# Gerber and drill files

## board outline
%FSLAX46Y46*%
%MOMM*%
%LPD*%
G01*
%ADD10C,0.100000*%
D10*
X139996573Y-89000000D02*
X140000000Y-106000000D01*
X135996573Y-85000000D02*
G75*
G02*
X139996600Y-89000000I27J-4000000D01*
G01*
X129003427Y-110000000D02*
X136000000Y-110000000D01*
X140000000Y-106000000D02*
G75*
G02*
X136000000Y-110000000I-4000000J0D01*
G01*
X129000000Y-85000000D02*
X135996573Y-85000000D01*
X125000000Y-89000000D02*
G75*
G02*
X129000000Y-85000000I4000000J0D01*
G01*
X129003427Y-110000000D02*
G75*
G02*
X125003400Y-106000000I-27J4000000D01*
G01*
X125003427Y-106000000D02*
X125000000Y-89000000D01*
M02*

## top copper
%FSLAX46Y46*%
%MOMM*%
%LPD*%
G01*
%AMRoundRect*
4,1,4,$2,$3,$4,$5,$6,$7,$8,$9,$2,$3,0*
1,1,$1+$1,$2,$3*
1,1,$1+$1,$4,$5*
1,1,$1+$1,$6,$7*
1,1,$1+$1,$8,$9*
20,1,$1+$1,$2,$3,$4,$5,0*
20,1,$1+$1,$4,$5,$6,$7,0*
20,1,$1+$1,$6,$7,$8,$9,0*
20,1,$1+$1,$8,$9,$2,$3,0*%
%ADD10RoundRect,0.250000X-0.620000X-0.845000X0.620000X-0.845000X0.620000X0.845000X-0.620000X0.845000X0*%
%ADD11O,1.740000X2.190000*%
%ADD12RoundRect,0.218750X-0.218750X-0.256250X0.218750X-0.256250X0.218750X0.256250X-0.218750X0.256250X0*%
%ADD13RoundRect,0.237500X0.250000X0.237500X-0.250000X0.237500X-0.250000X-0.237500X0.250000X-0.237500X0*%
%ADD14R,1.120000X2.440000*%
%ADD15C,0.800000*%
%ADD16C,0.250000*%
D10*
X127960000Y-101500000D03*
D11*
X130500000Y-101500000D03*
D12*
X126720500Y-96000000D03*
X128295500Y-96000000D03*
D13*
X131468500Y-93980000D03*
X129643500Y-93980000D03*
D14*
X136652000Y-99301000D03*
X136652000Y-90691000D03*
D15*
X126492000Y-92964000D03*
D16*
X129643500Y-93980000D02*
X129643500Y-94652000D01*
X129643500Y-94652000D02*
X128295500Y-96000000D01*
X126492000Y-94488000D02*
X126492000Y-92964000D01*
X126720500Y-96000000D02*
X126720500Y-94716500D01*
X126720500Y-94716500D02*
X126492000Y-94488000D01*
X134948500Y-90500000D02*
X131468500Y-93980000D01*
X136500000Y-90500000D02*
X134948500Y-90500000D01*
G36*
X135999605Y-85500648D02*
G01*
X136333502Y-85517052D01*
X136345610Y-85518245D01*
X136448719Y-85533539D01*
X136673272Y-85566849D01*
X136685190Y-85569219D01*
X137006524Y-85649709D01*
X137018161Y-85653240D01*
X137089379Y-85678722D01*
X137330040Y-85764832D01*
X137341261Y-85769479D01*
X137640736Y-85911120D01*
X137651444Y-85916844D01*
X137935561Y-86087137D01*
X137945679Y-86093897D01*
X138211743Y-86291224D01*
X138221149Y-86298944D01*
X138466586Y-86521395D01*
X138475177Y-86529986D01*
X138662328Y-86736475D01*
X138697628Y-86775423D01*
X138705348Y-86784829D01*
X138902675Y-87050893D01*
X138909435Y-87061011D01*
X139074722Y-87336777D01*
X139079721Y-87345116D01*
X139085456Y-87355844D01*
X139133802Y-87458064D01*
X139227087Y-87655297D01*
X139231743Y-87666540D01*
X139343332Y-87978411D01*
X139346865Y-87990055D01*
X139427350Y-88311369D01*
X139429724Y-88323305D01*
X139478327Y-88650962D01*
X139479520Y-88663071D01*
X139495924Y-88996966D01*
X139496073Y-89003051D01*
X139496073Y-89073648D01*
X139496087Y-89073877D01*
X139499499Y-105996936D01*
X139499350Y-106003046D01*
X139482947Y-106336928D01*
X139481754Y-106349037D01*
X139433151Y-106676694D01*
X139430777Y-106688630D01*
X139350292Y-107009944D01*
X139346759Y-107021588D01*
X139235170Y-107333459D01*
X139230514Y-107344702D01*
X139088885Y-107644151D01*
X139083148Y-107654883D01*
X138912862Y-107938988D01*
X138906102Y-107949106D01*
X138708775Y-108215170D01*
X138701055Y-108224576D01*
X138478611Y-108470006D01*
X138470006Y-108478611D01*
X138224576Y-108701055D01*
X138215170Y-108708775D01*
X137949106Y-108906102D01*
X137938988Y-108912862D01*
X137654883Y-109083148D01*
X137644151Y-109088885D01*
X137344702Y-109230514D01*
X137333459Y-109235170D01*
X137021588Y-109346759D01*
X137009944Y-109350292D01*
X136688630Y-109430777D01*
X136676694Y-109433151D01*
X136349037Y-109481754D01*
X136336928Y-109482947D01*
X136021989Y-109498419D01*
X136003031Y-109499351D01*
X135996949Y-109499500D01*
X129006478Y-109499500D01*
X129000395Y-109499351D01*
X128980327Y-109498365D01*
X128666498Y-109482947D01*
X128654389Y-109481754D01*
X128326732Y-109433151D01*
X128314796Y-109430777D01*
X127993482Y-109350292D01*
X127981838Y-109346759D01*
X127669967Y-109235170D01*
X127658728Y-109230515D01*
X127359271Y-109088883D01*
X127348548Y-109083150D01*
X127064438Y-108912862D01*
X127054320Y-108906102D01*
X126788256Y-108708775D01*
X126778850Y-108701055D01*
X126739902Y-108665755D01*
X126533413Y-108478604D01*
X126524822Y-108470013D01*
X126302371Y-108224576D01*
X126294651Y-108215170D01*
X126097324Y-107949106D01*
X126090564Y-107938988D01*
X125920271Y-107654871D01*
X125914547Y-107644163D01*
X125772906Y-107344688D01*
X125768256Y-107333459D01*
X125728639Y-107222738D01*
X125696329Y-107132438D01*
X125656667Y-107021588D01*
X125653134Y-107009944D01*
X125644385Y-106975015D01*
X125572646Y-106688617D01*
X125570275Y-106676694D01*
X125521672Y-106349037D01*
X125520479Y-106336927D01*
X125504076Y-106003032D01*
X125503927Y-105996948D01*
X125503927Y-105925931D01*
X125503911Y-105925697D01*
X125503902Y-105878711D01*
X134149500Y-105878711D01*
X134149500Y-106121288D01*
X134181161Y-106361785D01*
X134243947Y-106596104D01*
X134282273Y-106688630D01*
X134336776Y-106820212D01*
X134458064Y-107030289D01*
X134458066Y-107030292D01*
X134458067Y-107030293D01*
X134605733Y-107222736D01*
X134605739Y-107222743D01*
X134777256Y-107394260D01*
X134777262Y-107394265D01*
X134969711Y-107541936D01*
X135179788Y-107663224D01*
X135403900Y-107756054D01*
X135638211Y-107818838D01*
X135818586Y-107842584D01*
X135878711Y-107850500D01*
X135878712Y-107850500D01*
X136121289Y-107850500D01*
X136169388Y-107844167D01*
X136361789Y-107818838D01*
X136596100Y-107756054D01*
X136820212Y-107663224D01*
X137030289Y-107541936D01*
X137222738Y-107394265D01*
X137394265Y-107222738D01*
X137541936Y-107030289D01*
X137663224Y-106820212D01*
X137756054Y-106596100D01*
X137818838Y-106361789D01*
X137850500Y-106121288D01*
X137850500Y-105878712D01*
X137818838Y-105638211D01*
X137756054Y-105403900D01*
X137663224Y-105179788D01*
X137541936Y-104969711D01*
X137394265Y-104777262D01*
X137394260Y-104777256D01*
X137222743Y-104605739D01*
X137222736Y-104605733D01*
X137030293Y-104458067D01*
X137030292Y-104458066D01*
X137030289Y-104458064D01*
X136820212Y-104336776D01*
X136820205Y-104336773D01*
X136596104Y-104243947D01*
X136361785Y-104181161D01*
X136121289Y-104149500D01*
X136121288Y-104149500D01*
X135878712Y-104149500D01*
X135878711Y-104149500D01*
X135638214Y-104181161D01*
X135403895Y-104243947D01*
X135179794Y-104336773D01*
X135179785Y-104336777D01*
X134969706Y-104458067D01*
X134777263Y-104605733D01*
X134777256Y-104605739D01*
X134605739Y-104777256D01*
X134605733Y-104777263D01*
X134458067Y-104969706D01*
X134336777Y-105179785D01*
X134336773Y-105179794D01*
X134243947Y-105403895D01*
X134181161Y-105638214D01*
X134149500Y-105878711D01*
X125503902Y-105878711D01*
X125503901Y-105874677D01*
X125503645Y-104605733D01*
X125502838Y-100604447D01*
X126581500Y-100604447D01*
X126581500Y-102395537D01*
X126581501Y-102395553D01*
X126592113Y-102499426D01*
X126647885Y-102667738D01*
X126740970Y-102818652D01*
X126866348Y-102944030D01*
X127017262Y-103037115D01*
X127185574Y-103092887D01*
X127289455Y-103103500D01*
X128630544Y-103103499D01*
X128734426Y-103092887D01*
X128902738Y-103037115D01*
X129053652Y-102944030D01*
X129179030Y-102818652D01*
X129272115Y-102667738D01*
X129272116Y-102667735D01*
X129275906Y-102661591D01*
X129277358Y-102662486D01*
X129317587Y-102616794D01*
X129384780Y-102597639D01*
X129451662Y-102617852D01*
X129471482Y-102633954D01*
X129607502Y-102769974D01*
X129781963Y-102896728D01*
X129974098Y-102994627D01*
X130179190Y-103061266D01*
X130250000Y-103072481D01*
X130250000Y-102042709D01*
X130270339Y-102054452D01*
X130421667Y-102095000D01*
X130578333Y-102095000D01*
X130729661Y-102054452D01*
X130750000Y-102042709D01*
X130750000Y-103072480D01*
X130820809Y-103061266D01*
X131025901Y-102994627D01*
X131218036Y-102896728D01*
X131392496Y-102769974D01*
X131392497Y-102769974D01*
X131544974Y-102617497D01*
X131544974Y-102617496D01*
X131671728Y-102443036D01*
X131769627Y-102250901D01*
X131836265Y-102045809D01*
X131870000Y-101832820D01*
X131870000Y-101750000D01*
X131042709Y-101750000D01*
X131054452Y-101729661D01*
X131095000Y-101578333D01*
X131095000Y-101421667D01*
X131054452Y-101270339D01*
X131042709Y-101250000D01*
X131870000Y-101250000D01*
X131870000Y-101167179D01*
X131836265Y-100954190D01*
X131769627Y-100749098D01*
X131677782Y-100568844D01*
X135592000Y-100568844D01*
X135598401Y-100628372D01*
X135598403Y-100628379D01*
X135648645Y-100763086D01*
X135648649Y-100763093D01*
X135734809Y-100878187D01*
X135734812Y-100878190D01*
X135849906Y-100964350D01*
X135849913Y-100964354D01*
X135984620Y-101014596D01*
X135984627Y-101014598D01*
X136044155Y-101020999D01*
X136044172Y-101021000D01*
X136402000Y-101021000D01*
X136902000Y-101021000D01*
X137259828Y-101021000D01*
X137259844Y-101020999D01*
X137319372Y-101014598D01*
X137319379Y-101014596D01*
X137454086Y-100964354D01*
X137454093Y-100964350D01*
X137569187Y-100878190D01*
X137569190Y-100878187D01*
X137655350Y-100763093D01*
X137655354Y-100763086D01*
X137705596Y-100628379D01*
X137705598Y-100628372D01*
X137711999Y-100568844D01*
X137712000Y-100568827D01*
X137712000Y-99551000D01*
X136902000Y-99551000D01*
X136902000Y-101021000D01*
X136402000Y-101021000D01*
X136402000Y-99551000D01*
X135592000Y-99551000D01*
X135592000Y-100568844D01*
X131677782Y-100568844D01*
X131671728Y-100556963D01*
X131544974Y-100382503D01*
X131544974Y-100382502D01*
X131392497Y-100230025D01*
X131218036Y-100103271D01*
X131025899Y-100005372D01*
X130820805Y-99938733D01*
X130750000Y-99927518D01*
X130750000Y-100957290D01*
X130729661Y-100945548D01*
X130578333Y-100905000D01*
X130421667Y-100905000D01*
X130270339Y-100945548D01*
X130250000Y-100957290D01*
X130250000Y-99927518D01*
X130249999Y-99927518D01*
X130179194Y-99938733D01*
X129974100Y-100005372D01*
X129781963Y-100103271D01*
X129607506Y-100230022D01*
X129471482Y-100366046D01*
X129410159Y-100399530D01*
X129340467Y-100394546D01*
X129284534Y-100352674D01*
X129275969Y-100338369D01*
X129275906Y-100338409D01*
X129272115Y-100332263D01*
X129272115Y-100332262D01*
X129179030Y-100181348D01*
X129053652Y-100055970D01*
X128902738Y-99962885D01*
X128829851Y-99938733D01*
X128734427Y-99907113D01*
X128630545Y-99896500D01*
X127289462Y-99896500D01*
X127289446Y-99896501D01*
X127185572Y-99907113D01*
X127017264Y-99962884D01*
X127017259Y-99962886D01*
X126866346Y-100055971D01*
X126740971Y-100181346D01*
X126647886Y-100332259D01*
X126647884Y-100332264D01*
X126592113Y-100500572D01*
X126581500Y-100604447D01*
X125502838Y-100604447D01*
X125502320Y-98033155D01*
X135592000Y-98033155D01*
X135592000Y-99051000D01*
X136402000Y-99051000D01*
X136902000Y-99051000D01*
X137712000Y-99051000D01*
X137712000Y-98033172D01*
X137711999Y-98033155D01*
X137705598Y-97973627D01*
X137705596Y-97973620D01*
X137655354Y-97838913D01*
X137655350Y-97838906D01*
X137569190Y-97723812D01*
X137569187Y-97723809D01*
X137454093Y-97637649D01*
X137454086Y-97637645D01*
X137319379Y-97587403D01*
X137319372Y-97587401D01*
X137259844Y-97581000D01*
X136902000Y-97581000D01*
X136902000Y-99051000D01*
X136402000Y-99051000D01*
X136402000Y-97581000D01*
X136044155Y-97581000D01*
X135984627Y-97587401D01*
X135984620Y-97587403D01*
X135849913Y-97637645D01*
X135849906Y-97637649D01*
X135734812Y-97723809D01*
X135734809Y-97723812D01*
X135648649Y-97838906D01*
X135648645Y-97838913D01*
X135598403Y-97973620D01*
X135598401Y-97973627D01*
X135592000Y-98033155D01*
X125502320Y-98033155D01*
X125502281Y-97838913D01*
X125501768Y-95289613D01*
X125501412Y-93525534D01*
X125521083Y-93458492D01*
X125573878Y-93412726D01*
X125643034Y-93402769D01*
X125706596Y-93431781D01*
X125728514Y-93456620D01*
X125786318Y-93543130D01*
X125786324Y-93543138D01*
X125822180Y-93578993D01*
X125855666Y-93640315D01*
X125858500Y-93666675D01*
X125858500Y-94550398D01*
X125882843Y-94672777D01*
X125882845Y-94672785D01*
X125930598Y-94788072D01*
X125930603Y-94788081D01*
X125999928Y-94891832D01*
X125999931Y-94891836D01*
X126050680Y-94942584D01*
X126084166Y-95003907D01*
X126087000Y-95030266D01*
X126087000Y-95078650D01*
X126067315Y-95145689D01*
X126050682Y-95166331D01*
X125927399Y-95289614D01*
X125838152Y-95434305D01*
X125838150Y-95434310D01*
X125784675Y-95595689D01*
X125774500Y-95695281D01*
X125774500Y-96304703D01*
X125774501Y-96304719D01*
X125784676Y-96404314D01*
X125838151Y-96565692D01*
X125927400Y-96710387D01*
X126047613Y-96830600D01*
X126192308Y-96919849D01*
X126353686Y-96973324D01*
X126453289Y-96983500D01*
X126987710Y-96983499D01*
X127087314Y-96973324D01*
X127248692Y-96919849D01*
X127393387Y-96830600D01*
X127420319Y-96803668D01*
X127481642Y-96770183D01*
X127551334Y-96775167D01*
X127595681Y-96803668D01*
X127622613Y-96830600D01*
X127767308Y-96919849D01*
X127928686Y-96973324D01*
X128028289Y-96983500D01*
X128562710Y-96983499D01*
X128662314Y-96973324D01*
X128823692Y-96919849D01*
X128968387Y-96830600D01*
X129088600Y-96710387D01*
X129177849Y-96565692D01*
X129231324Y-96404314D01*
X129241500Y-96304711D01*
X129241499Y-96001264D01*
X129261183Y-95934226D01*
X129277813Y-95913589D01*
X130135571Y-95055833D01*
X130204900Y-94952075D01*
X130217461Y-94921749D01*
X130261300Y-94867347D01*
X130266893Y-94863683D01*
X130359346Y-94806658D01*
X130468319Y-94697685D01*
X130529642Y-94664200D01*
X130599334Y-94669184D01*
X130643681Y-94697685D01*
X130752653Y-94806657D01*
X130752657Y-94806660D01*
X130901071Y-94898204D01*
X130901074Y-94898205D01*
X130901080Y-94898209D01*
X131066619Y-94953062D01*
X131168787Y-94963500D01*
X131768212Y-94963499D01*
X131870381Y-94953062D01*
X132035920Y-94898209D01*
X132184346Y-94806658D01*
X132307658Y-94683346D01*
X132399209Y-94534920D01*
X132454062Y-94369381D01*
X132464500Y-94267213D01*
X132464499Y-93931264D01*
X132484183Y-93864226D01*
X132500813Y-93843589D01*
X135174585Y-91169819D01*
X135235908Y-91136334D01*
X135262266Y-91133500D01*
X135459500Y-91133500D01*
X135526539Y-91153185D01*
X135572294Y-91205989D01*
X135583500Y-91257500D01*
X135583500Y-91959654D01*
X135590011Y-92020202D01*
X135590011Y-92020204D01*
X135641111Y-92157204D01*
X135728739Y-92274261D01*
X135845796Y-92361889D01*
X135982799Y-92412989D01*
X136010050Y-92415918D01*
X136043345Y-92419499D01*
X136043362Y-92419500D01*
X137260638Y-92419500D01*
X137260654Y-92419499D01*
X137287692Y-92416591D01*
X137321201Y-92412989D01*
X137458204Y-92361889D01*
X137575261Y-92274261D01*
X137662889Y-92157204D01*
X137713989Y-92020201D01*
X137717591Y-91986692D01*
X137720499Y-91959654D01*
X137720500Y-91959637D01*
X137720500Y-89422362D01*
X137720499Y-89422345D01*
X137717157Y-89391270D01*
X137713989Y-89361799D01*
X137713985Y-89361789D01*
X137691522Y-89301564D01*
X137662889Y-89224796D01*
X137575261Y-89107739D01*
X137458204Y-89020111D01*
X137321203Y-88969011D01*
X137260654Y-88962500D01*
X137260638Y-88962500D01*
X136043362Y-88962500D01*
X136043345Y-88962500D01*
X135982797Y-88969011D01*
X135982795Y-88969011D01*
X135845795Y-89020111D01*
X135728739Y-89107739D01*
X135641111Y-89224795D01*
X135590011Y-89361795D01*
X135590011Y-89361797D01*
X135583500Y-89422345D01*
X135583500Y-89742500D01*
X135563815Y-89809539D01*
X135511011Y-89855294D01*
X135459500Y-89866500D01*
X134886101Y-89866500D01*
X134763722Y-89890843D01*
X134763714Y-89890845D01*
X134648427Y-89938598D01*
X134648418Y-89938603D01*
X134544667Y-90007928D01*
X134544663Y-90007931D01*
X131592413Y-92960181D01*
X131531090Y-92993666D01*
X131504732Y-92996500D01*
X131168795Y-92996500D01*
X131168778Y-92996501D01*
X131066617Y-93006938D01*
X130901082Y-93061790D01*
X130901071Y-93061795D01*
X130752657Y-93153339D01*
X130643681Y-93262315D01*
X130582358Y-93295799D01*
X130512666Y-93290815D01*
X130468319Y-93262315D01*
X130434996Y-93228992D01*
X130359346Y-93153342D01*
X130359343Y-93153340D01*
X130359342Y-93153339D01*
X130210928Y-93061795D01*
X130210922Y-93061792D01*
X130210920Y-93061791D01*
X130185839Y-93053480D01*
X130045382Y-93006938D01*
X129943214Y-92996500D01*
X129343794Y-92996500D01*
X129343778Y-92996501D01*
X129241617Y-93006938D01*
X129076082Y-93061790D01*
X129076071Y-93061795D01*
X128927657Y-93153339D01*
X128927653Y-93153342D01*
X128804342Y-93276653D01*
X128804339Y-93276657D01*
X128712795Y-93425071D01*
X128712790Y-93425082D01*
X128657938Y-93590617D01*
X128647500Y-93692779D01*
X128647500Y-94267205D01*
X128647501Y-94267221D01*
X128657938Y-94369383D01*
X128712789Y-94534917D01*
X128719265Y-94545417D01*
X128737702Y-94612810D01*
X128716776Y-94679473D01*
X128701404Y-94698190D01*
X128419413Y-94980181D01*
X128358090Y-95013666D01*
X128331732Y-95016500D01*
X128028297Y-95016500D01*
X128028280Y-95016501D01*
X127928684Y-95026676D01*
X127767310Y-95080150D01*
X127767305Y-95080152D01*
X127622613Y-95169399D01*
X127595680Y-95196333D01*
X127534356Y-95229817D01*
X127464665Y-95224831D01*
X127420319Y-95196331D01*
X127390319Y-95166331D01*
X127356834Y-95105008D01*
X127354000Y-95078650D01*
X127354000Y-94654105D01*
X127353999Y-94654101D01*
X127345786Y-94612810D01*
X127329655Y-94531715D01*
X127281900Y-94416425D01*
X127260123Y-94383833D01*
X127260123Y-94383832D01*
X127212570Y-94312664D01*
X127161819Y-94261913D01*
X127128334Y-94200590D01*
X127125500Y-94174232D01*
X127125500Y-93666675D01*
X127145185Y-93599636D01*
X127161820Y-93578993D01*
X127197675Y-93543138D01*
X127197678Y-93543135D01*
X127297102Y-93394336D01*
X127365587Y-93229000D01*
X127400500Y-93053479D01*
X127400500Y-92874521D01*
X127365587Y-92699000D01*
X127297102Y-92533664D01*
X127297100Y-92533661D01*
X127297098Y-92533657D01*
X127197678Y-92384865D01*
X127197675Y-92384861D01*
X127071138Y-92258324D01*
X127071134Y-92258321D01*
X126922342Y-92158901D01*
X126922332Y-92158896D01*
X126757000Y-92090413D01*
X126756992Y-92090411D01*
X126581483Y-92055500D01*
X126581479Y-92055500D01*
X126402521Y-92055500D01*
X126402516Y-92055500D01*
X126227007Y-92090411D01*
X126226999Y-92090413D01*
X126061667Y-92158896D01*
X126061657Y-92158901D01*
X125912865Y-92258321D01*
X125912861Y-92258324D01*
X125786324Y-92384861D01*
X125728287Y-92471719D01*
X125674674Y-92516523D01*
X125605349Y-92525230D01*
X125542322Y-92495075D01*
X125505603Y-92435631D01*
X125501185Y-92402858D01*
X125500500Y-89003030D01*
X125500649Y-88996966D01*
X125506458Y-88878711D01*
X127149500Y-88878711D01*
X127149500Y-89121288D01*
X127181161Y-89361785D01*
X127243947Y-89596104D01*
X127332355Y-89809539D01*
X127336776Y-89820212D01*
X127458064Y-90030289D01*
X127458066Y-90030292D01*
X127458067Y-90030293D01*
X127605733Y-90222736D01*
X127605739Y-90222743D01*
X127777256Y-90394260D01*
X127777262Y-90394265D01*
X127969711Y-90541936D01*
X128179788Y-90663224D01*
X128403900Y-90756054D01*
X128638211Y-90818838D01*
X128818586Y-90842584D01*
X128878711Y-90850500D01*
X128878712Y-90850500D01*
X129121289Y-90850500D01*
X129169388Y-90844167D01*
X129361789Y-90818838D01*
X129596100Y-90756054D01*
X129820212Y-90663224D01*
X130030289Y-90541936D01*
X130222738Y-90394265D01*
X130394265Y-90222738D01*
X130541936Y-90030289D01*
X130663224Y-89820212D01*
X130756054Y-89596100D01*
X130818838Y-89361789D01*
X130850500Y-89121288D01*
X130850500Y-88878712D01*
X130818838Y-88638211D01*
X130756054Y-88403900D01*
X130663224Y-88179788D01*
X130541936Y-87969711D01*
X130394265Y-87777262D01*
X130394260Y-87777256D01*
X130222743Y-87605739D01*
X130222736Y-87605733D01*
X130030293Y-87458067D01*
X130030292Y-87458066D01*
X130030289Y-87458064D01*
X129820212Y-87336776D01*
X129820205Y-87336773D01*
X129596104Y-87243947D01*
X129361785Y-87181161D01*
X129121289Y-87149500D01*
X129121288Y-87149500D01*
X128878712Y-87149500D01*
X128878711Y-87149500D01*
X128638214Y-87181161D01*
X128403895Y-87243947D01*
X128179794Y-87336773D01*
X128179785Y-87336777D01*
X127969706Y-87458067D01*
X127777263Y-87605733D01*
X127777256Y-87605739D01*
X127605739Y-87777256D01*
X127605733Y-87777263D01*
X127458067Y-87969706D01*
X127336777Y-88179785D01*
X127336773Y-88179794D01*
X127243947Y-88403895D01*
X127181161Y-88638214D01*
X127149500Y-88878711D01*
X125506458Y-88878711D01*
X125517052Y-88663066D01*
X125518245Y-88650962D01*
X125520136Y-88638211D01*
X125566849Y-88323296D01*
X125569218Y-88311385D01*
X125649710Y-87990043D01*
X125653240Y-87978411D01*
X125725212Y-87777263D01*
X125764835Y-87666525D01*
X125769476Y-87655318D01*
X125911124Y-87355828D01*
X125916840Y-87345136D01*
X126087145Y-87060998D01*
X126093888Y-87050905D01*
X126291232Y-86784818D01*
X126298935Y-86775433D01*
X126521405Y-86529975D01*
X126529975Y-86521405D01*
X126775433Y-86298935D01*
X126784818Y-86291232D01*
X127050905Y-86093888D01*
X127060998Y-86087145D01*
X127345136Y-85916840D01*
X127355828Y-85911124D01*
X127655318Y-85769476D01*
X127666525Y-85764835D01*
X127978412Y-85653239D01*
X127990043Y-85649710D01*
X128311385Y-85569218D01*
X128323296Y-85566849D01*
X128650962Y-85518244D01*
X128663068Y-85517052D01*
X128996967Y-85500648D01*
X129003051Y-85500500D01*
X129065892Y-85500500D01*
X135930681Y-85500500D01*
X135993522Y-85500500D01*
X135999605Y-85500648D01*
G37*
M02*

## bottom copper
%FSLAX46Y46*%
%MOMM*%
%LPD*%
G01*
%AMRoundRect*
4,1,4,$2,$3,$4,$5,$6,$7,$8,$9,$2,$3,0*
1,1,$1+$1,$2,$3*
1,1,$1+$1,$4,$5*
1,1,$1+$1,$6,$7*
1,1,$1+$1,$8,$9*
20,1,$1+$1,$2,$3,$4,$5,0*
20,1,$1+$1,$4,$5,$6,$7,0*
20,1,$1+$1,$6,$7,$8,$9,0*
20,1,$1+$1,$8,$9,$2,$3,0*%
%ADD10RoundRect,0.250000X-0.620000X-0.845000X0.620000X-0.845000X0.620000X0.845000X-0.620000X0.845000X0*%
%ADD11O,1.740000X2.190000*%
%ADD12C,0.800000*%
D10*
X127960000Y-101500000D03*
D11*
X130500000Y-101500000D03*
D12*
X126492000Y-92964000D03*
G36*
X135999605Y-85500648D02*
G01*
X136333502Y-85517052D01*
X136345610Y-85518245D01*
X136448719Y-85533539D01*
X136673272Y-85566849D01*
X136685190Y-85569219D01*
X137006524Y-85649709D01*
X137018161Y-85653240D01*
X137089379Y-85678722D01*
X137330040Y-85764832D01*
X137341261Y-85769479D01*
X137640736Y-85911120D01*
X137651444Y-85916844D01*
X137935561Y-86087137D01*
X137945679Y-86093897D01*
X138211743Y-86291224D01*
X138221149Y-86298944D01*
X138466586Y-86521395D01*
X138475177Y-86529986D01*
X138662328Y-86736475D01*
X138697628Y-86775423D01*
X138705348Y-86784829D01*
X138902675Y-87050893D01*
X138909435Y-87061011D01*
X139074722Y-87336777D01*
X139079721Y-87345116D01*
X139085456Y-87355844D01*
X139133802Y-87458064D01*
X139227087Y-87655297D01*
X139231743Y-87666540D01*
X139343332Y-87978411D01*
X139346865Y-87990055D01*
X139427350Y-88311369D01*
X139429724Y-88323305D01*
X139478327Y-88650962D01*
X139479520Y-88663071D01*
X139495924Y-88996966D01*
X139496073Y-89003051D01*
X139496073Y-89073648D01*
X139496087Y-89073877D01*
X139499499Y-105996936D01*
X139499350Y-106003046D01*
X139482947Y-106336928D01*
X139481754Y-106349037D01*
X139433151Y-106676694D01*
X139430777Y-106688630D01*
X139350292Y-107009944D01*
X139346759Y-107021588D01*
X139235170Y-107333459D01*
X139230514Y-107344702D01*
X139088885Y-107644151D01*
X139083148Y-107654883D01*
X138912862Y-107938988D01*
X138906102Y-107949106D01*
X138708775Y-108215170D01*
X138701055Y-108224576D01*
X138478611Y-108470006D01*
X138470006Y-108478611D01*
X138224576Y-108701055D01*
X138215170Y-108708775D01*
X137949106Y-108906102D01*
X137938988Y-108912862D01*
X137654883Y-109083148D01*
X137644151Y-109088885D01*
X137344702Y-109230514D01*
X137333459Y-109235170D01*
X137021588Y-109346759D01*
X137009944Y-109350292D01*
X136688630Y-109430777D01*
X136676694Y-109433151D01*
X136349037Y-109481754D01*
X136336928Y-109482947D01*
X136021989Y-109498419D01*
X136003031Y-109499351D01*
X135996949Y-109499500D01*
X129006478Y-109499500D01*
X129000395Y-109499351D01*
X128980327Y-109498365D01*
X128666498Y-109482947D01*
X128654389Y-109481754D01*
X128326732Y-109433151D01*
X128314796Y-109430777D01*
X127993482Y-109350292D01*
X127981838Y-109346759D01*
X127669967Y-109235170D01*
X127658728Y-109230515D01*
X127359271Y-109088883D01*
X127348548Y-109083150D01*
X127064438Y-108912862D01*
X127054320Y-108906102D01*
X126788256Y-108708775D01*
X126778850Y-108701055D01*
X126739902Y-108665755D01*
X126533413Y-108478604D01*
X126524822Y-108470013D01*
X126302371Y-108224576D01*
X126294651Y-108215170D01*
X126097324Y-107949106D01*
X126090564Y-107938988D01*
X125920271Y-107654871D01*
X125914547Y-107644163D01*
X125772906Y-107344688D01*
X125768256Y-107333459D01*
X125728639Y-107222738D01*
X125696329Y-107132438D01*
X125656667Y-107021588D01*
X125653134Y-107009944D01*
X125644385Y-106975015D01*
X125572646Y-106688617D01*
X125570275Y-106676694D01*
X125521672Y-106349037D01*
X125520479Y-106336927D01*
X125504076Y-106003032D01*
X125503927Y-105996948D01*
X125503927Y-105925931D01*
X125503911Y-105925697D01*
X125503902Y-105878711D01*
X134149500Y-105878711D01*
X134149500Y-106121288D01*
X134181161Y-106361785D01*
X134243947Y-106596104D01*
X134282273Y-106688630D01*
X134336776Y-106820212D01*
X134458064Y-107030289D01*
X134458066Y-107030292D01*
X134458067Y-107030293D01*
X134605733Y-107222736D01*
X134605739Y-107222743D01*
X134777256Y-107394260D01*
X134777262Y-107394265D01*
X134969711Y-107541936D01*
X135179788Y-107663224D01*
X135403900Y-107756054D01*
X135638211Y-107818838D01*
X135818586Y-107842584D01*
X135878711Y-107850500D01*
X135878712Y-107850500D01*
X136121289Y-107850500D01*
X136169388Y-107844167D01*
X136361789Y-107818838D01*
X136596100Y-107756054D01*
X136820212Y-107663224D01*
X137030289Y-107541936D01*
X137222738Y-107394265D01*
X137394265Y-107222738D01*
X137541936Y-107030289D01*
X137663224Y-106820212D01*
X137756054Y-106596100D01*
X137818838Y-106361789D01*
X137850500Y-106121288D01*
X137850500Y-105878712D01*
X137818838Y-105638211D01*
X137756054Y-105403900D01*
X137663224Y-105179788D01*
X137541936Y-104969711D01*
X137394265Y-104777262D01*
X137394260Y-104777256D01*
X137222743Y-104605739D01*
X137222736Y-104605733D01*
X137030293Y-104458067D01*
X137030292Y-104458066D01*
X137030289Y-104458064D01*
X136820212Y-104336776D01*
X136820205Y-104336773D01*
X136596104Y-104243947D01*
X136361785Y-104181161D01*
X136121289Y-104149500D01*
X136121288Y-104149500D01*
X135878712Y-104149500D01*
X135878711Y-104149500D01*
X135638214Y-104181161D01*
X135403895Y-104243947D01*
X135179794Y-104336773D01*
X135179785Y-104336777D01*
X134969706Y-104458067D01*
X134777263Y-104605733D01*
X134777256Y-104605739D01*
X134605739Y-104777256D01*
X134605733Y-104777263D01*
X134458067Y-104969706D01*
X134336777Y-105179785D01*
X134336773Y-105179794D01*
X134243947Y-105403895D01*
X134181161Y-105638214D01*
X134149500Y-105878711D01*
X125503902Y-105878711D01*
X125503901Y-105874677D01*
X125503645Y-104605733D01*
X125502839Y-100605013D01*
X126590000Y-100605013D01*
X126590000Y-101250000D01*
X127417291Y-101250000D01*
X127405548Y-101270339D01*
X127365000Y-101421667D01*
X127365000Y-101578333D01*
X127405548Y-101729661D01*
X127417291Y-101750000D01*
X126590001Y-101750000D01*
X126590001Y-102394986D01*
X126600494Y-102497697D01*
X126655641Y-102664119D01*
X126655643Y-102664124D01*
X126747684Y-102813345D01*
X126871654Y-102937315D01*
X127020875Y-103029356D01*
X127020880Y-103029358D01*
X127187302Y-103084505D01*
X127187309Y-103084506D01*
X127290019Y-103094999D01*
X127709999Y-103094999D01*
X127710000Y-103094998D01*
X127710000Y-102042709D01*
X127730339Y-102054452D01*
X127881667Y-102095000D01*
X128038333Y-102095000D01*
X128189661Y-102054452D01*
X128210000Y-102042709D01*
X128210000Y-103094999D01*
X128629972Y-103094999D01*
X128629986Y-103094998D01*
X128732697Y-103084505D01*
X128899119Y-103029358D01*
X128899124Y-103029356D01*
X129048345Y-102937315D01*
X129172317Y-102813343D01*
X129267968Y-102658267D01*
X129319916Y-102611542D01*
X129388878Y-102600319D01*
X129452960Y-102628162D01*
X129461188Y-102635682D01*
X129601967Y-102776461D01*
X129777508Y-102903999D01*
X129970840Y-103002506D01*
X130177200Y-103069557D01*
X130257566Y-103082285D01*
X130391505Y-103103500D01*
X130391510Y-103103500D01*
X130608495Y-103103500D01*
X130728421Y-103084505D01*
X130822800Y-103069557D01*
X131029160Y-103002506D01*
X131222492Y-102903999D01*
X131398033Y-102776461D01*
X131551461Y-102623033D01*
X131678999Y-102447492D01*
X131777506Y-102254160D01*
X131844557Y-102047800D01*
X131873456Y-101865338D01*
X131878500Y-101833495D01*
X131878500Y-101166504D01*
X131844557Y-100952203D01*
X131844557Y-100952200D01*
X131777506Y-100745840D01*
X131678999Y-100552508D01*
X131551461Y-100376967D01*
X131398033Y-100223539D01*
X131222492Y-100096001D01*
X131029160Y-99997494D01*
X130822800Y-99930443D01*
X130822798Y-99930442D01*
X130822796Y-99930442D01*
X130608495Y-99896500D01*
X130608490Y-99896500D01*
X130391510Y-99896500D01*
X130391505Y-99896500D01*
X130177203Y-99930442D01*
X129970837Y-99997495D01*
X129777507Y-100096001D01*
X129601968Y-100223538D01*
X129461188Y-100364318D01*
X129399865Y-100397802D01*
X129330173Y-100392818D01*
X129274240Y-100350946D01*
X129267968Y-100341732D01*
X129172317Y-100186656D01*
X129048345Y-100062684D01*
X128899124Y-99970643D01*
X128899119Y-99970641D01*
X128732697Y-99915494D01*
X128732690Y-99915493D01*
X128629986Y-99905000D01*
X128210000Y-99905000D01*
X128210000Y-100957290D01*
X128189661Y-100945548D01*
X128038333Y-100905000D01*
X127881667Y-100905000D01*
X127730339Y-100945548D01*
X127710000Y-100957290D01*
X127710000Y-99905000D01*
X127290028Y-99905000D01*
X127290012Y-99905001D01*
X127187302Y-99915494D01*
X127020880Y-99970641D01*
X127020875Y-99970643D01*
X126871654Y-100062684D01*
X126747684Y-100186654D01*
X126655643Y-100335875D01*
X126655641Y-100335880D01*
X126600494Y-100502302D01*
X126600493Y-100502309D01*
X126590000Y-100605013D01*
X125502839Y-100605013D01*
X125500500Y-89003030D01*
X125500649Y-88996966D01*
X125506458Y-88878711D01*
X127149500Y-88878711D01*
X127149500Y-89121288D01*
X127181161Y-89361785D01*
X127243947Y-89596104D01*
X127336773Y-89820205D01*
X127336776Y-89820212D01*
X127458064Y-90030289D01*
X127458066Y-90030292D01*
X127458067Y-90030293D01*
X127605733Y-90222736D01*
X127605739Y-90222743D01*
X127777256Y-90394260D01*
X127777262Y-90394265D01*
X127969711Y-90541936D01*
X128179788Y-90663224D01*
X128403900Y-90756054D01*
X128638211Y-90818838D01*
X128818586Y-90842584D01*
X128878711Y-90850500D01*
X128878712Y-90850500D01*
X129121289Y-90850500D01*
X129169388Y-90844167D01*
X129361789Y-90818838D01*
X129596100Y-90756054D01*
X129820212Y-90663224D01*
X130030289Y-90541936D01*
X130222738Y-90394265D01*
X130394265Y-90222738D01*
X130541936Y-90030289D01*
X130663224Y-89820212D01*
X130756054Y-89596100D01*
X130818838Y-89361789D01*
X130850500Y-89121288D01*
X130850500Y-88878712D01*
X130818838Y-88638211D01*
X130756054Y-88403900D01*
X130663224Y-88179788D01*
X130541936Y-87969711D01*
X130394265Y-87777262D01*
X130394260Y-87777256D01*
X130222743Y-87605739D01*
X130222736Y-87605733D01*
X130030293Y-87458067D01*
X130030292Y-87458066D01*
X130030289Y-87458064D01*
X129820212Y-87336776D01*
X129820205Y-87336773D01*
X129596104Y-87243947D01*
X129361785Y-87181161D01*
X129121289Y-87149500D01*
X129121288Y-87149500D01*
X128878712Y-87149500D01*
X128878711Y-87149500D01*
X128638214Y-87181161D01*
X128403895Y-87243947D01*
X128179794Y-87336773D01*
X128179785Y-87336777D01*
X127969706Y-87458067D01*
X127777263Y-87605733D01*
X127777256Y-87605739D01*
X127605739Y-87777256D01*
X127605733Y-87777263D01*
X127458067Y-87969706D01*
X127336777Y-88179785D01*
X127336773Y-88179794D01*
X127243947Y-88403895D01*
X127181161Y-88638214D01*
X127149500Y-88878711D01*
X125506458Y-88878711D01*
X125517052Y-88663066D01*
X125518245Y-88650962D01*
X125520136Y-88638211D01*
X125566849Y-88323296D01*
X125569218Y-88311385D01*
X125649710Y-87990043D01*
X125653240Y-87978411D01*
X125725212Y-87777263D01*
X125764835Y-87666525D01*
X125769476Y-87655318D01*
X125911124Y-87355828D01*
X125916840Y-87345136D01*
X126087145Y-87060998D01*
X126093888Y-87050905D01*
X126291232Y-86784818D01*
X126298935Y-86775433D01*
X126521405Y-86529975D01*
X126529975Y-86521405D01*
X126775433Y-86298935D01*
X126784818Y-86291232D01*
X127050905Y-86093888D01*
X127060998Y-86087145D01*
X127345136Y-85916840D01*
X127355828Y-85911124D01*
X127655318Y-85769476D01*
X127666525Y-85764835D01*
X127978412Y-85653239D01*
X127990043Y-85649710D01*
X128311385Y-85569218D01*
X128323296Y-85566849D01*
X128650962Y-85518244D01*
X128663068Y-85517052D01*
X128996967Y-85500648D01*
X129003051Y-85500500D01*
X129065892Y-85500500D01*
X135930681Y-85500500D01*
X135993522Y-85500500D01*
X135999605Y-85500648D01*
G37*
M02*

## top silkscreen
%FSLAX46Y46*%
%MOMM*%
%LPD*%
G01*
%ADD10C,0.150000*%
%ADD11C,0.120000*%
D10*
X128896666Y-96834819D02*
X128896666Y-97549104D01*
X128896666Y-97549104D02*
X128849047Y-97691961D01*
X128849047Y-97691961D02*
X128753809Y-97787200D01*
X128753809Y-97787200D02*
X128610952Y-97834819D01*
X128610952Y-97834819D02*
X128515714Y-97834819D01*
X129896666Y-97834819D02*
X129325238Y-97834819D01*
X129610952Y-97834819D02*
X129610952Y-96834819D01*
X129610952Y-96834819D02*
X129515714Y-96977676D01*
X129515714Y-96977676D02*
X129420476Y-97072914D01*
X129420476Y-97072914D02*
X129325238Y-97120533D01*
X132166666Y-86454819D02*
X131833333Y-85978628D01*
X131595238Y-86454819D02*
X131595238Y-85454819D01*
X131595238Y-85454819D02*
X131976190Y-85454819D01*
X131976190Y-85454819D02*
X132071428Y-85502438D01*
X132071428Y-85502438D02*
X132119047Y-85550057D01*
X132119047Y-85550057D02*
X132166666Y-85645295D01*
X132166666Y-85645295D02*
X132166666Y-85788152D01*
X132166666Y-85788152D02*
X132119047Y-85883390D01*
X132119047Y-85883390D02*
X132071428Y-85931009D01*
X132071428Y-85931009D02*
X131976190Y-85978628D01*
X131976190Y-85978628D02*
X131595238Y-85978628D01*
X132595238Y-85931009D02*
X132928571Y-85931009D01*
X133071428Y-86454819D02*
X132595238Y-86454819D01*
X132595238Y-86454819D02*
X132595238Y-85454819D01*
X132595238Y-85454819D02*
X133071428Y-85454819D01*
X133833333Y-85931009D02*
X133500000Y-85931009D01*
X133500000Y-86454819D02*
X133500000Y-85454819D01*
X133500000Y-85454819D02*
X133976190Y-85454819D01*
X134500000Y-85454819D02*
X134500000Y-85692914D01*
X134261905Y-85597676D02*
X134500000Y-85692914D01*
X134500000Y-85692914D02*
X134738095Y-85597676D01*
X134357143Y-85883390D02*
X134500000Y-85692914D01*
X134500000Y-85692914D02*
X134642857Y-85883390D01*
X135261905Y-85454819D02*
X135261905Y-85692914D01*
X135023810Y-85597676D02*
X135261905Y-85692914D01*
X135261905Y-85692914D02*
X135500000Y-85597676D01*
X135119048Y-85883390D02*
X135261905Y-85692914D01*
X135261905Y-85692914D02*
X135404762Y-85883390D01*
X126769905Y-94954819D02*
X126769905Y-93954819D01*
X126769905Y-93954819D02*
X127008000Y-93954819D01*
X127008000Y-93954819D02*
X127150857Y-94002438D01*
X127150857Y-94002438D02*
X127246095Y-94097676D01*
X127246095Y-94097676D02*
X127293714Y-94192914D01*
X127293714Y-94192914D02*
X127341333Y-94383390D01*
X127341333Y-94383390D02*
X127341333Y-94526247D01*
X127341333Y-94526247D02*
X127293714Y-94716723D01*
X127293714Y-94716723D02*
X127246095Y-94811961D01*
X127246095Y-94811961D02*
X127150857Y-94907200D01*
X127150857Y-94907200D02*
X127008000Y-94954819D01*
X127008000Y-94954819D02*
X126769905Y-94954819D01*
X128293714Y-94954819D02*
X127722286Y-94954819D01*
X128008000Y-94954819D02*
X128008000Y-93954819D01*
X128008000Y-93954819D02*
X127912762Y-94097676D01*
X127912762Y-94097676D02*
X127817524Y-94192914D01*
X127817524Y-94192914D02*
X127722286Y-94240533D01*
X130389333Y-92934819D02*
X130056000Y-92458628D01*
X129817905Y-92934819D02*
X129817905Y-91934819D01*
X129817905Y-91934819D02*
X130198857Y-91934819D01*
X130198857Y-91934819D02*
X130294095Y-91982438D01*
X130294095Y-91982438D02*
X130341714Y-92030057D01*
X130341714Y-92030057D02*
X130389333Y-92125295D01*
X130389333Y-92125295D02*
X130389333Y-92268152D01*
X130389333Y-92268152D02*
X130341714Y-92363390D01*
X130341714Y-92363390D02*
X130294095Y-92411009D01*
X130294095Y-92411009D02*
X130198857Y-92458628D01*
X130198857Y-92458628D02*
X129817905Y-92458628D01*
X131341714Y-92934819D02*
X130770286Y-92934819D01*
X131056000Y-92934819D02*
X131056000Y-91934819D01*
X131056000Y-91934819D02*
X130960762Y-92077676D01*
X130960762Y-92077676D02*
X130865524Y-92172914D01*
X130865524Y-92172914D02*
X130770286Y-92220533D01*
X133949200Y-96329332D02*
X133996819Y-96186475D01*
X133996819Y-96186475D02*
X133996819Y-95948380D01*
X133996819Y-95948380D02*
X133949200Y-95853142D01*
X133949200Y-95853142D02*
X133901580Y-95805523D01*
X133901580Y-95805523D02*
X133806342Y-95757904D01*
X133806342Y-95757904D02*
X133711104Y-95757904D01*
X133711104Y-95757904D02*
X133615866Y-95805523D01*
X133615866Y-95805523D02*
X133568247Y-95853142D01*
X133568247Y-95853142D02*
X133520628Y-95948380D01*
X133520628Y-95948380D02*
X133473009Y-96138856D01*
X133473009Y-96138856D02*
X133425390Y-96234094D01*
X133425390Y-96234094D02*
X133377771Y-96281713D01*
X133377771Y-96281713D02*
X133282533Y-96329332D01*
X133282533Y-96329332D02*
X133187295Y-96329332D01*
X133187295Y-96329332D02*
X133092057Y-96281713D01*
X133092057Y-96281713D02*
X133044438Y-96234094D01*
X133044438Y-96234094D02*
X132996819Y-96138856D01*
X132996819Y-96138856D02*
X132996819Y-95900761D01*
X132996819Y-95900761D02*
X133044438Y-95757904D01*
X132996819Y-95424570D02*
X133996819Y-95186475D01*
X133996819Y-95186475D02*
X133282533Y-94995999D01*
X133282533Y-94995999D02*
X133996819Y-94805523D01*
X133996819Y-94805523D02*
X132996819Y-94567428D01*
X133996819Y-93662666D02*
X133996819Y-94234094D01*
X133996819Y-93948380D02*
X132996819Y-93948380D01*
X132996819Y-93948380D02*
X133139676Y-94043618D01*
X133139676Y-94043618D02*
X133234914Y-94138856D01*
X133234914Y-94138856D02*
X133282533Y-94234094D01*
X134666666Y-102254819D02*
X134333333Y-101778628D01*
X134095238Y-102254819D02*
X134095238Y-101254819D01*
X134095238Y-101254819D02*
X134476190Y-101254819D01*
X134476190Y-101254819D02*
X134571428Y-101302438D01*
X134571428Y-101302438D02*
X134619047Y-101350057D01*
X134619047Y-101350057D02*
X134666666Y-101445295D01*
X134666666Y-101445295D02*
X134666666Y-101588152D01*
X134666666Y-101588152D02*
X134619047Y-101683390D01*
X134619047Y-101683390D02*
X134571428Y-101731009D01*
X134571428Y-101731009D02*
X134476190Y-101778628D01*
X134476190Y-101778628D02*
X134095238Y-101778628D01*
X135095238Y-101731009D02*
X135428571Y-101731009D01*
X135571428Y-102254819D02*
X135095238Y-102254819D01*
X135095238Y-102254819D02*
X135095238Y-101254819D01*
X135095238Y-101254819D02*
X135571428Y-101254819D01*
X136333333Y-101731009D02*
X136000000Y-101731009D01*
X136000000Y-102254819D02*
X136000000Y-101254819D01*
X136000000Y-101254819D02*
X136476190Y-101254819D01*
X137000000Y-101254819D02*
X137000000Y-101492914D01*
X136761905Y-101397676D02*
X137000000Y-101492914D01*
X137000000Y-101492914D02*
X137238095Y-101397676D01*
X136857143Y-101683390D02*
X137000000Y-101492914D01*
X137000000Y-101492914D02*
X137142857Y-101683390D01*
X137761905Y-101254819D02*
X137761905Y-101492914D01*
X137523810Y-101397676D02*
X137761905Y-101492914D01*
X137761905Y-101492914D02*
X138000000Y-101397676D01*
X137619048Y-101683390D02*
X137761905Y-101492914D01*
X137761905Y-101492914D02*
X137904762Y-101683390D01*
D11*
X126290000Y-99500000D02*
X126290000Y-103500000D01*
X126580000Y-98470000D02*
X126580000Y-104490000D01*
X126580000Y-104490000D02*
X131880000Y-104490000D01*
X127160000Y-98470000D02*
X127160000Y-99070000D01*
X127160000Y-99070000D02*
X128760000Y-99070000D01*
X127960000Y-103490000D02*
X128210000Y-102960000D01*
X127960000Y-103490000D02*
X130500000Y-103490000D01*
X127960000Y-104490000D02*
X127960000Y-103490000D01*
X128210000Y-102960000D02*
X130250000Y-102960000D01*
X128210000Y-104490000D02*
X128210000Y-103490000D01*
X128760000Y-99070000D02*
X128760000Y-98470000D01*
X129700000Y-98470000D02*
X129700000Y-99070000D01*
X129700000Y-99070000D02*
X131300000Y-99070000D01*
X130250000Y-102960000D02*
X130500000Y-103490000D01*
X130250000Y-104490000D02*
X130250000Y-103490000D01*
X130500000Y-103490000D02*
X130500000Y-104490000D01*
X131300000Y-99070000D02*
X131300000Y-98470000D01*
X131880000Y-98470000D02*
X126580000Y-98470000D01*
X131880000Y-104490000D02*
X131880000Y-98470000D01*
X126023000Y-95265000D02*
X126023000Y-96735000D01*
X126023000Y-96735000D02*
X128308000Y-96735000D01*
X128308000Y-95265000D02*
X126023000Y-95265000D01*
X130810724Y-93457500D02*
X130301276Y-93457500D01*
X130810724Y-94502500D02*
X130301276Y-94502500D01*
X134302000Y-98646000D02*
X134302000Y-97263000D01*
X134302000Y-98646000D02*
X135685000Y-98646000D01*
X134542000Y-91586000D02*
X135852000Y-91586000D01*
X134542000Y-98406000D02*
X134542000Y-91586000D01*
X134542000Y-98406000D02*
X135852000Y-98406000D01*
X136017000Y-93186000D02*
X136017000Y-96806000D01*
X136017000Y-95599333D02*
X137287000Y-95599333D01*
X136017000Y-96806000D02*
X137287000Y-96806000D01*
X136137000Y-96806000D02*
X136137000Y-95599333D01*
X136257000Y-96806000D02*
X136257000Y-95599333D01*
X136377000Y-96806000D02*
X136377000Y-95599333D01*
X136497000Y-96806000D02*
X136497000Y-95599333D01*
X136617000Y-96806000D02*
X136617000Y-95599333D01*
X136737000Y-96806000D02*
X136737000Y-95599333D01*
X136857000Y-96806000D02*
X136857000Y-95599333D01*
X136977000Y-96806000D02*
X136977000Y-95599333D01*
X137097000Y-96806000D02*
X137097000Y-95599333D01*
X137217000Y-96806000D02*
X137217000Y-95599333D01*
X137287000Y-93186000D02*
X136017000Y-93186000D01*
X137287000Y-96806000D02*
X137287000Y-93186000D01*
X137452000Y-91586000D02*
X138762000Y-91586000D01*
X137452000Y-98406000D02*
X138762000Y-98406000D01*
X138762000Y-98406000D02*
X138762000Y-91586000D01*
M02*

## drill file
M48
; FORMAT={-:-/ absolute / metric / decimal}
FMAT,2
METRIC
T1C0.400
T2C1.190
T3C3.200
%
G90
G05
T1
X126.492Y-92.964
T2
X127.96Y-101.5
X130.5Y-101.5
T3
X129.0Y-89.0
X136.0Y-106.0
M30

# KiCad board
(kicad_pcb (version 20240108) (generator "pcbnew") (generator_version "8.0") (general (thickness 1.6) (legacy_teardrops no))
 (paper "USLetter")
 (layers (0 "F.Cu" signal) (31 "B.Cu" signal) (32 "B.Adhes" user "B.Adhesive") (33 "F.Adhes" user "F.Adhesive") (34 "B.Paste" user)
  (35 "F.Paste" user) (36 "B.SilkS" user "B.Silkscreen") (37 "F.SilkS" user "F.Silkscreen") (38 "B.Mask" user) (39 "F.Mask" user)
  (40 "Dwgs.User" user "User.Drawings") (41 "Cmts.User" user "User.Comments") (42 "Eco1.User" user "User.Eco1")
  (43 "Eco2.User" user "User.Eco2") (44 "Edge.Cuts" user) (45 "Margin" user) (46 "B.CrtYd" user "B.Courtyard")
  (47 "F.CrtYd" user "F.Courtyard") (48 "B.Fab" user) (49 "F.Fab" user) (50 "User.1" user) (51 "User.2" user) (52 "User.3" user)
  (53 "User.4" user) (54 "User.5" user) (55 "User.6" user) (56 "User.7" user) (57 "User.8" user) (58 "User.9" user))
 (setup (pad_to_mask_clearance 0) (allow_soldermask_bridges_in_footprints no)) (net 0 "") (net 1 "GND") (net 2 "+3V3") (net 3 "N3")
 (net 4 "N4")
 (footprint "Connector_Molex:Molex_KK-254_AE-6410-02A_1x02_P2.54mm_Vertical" (layer "F.Cu") (at 127.96 101.5)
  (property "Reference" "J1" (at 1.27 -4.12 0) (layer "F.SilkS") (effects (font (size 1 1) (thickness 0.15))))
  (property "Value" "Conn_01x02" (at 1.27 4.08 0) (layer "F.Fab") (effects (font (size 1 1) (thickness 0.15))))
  (fp_line (start -1.67 -2) (end -1.67 2) (stroke (width 0.12) (type solid)) (layer "F.SilkS"))
  (fp_line (start -1.38 -3.03) (end -1.38 2.99) (stroke (width 0.12) (type solid)) (layer "F.SilkS"))
  (fp_line (start -1.38 2.99) (end 3.92 2.99) (stroke (width 0.12) (type solid)) (layer "F.SilkS"))
  (fp_line (start -0.8 -3.03) (end -0.8 -2.43) (stroke (width 0.12) (type solid)) (layer "F.SilkS"))
  (fp_line (start -0.8 -2.43) (end 0.8 -2.43) (stroke (width 0.12) (type solid)) (layer "F.SilkS"))
  (fp_line (start 0 1.99) (end 0.25 1.46) (stroke (width 0.12) (type solid)) (layer "F.SilkS"))
  (fp_line (start 0 1.99) (end 2.54 1.99) (stroke (width 0.12) (type solid)) (layer "F.SilkS"))
  (fp_line (start 0 2.99) (end 0 1.99) (stroke (width 0.12) (type solid)) (layer "F.SilkS"))
  (fp_line (start 0.25 1.46) (end 2.29 1.46) (stroke (width 0.12) (type solid)) (layer "F.SilkS"))
  (fp_line (start 0.25 2.99) (end 0.25 1.99) (stroke (width 0.12) (type solid)) (layer "F.SilkS"))
  (fp_line (start 0.8 -2.43) (end 0.8 -3.03) (stroke (width 0.12) (type solid)) (layer "F.SilkS"))
  (fp_line (start 1.74 -3.03) (end 1.74 -2.43) (stroke (width 0.12) (type solid)) (layer "F.SilkS"))
  (fp_line (start 1.74 -2.43) (end 3.34 -2.43) (stroke (width 0.12) (type solid)) (layer "F.SilkS"))
  (fp_line (start 2.29 1.46) (end 2.54 1.99) (stroke (width 0.12) (type solid)) (layer "F.SilkS"))
  (fp_line (start 2.29 2.99) (end 2.29 1.99) (stroke (width 0.12) (type solid)) (layer "F.SilkS"))
  (fp_line (start 2.54 1.99) (end 2.54 2.99) (stroke (width 0.12) (type solid)) (layer "F.SilkS"))
  (fp_line (start 3.34 -2.43) (end 3.34 -3.03) (stroke (width 0.12) (type solid)) (layer "F.SilkS"))
  (fp_line (start 3.92 -3.03) (end -1.38 -3.03) (stroke (width 0.12) (type solid)) (layer "F.SilkS"))
  (fp_line (start 3.92 2.99) (end 3.92 -3.03) (stroke (width 0.12) (type solid)) (layer "F.SilkS"))
  (pad "1" thru_hole roundrect (at 0 0) (size 1.74 2.19) (drill 1.19) (layers "*.Cu" "*.Mask") (remove_unused_layers no)
   (roundrect_rratio 0.143678) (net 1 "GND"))
  (pad "2" thru_hole oval (at 2.54 0) (size 1.74 2.19) (drill 1.19) (layers "*.Cu" "*.Mask") (remove_unused_layers no) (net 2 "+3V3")))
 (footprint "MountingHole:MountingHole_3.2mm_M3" (layer "F.Cu") (at 129 89)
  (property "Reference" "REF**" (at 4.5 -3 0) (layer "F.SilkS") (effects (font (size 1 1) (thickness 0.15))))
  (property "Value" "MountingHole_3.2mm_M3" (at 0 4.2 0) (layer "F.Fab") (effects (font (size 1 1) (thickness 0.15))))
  (pad "" np_thru_hole circle (at 0 0) (size 3.2 3.2) (drill 3.2) (layers "*.Cu" "*.Mask")))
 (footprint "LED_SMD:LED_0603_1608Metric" (layer "F.Cu") (at 127.508 96)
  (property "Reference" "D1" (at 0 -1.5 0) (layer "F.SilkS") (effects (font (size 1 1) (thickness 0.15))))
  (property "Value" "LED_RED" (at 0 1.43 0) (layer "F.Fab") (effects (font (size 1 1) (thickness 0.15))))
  (fp_line (start -1.485 -0.735) (end -1.485 0.735) (stroke (width 0.12) (type solid)) (layer "F.SilkS"))
  (fp_line (start -1.485 0.735) (end 0.8 0.735) (stroke (width 0.12) (type solid)) (layer "F.SilkS"))
  (fp_line (start 0.8 -0.735) (end -1.485 -0.735) (stroke (width 0.12) (type solid)) (layer "F.SilkS"))
  (pad "1" smd roundrect (at -0.7875 0) (size 0.875 0.95) (layers "F.Cu" "F.Paste" "F.Mask") (roundrect_rratio 0.25) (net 1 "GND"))
  (pad "2" smd roundrect (at 0.7875 0) (size 0.875 0.95) (layers "F.Cu" "F.Paste" "F.Mask") (roundrect_rratio 0.25) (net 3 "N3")))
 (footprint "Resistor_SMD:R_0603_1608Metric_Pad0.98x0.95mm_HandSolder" (layer "F.Cu") (at 130.556 93.98 180)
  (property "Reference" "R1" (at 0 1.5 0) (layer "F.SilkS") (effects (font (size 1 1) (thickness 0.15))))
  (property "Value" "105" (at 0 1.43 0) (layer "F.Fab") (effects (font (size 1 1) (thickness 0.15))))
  (fp_line (start -0.254724 0.5225) (end 0.254724 0.5225) (stroke (width 0.12) (type solid)) (layer "F.SilkS"))
  (fp_line (start -0.254724 -0.5225) (end 0.254724 -0.5225) (stroke (width 0.12) (type solid)) (layer "F.SilkS"))
  (pad "1" smd roundrect (at -0.9125 0 180) (size 0.975 0.95) (layers "F.Cu" "F.Paste" "F.Mask") (roundrect_rratio 0.25) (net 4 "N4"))
  (pad "2" smd roundrect (at 0.9125 0 180) (size 0.975 0.95) (layers "F.Cu" "F.Paste" "F.Mask") (roundrect_rratio 0.25) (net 3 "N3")))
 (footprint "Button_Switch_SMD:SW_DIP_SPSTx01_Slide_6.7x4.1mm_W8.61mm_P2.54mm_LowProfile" (layer "F.Cu") (at 136.652 94.996 90)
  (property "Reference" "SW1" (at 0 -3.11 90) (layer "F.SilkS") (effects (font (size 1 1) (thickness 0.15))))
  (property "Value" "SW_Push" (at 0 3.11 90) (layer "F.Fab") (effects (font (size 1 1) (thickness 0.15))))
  (fp_line (start -3.65 -2.35) (end -2.267 -2.35) (stroke (width 0.12) (type solid)) (layer "F.SilkS"))
  (fp_line (start -3.65 -2.35) (end -3.65 -0.967) (stroke (width 0.12) (type solid)) (layer "F.SilkS"))
  (fp_line (start 3.41 -2.11) (end 3.41 -0.8) (stroke (width 0.12) (type solid)) (layer "F.SilkS"))
  (fp_line (start -3.41 -2.11) (end 3.41 -2.11) (stroke (width 0.12) (type solid)) (layer "F.SilkS"))
  (fp_line (start -3.41 -2.11) (end -3.41 -0.8) (stroke (width 0.12) (type solid)) (layer "F.SilkS"))
  (fp_line (start 1.81 -0.635) (end -1.81 -0.635) (stroke (width 0.12) (type solid)) (layer "F.SilkS"))
  (fp_line (start -0.603333 -0.635) (end -0.603333 0.635) (stroke (width 0.12) (type solid)) (layer "F.SilkS"))
  (fp_line (start -1.81 -0.635) (end -1.81 0.635) (stroke (width 0.12) (type solid)) (layer "F.SilkS"))
  (fp_line (start -1.81 -0.515) (end -0.603333 -0.515) (stroke (width 0.12) (type solid)) (layer "F.SilkS"))
  (fp_line (start -1.81 -0.395) (end -0.603333 -0.395) (stroke (width 0.12) (type solid)) (layer "F.SilkS"))
  (fp_line (start -1.81 -0.275) (end -0.603333 -0.275) (stroke (width 0.12) (type solid)) (layer "F.SilkS"))
  (fp_line (start -1.81 -0.155) (end -0.603333 -0.155) (stroke (width 0.12) (type solid)) (layer "F.SilkS"))
  (fp_line (start -1.81 -0.035) (end -0.603333 -0.035) (stroke (width 0.12) (type solid)) (layer "F.SilkS"))
  (fp_line (start -1.81 0.085) (end -0.603333 0.085) (stroke (width 0.12) (type solid)) (layer "F.SilkS"))
  (fp_line (start -1.81 0.205) (end -0.603333 0.205) (stroke (width 0.12) (type solid)) (layer "F.SilkS"))
  (fp_line (start -1.81 0.325) (end -0.603333 0.325) (stroke (width 0.12) (type solid)) (layer "F.SilkS"))
  (fp_line (start -1.81 0.445) (end -0.603333 0.445) (stroke (width 0.12) (type solid)) (layer "F.SilkS"))
  (fp_line (start -1.81 0.565) (end -0.603333 0.565) (stroke (width 0.12) (type solid)) (layer "F.SilkS"))
  (fp_line (start 1.81 0.635) (end 1.81 -0.635) (stroke (width 0.12) (type solid)) (layer "F.SilkS"))
  (fp_line (start -1.81 0.635) (end 1.81 0.635) (stroke (width 0.12) (type solid)) (layer "F.SilkS"))
  (fp_line (start 3.41 0.8) (end 3.41 2.11) (stroke (width 0.12) (type solid)) (layer "F.SilkS"))
  (fp_line (start -3.41 0.8) (end -3.41 2.11) (stroke (width 0.12) (type solid)) (layer "F.SilkS"))
  (fp_line (start -3.41 2.11) (end 3.41 2.11) (stroke (width 0.12) (type solid)) (layer "F.SilkS"))
  (pad "1" smd rect (at -4.305 0 90) (size 2.44 1.12) (layers "F.Cu" "F.Paste" "F.Mask") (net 2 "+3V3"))
  (pad "2" smd rect (at 4.305 0 90) (size 2.44 1.12) (layers "F.Cu" "F.Paste" "F.Mask") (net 4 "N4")))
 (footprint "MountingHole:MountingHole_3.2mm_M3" (layer "F.Cu") (at 136 106)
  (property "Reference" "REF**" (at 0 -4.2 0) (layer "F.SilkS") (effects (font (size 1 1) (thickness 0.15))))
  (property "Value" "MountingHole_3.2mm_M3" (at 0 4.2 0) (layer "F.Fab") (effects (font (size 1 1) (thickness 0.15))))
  (pad "" np_thru_hole circle (at 0 0) (size 3.2 3.2) (drill 3.2) (layers "*.Cu" "*.Mask")))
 (gr_line (start 139.996573 89) (end 140 106) (stroke (width 0.1) (type default)) (layer "Edge.Cuts"))
 (gr_arc (start 135.996573 85) (mid 138.825 86.171573) (end 139.996573 89) (stroke (width 0.1) (type default)) (layer "Edge.Cuts"))
 (gr_line (start 129.003427 110) (end 136 110) (stroke (width 0.1) (type default)) (layer "Edge.Cuts"))
 (gr_arc (start 140 106) (mid 138.828427 108.828427) (end 136 110) (stroke (width 0.1) (type default)) (layer "Edge.Cuts"))
 (gr_line (start 129 85) (end 135.996573 85) (stroke (width 0.1) (type default)) (layer "Edge.Cuts"))
 (gr_arc (start 125 89) (mid 126.171573 86.171573) (end 129 85) (stroke (width 0.1) (type default)) (layer "Edge.Cuts"))
 (gr_arc (start 129.003427 110) (mid 126.175 108.828427) (end 125.003427 106) (stroke (width 0.1) (type default)) (layer "Edge.Cuts"))
 (gr_line (start 125.003427 106) (end 125 89) (stroke (width 0.1) (type default)) (layer "Edge.Cuts"))
 (segment (start 129.6435 93.98) (end 129.6435 94.652) (width 0.25) (layer "F.Cu") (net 3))
 (segment (start 129.6435 94.652) (end 128.2955 96) (width 0.25) (layer "F.Cu") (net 3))
 (segment (start 126.492 94.488) (end 126.492 92.964) (width 0.25) (layer "F.Cu") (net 1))
 (segment (start 126.7205 96) (end 126.7205 94.7165) (width 0.25) (layer "F.Cu") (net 1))
 (segment (start 126.7205 94.7165) (end 126.492 94.488) (width 0.25) (layer "F.Cu") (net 1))
 (via (at 126.492 92.964) (size 0.8) (drill 0.4) (layers "F.Cu" "B.Cu") (free yes) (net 1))
 (segment (start 134.9485 90.5) (end 131.4685 93.98) (width 0.25) (layer "F.Cu") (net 4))
 (segment (start 136.5 90.5) (end 134.9485 90.5) (width 0.25) (layer "F.Cu") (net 4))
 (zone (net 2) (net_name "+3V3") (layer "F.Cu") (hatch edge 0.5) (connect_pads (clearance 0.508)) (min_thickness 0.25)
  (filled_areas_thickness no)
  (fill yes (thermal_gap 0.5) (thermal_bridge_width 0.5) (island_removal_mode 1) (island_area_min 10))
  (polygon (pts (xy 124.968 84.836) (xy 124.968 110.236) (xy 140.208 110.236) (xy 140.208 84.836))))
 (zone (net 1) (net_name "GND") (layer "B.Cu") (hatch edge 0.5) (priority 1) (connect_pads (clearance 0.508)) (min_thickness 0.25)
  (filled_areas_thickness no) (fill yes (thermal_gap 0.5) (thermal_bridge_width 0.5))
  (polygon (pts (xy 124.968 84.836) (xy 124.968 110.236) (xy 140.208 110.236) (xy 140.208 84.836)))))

